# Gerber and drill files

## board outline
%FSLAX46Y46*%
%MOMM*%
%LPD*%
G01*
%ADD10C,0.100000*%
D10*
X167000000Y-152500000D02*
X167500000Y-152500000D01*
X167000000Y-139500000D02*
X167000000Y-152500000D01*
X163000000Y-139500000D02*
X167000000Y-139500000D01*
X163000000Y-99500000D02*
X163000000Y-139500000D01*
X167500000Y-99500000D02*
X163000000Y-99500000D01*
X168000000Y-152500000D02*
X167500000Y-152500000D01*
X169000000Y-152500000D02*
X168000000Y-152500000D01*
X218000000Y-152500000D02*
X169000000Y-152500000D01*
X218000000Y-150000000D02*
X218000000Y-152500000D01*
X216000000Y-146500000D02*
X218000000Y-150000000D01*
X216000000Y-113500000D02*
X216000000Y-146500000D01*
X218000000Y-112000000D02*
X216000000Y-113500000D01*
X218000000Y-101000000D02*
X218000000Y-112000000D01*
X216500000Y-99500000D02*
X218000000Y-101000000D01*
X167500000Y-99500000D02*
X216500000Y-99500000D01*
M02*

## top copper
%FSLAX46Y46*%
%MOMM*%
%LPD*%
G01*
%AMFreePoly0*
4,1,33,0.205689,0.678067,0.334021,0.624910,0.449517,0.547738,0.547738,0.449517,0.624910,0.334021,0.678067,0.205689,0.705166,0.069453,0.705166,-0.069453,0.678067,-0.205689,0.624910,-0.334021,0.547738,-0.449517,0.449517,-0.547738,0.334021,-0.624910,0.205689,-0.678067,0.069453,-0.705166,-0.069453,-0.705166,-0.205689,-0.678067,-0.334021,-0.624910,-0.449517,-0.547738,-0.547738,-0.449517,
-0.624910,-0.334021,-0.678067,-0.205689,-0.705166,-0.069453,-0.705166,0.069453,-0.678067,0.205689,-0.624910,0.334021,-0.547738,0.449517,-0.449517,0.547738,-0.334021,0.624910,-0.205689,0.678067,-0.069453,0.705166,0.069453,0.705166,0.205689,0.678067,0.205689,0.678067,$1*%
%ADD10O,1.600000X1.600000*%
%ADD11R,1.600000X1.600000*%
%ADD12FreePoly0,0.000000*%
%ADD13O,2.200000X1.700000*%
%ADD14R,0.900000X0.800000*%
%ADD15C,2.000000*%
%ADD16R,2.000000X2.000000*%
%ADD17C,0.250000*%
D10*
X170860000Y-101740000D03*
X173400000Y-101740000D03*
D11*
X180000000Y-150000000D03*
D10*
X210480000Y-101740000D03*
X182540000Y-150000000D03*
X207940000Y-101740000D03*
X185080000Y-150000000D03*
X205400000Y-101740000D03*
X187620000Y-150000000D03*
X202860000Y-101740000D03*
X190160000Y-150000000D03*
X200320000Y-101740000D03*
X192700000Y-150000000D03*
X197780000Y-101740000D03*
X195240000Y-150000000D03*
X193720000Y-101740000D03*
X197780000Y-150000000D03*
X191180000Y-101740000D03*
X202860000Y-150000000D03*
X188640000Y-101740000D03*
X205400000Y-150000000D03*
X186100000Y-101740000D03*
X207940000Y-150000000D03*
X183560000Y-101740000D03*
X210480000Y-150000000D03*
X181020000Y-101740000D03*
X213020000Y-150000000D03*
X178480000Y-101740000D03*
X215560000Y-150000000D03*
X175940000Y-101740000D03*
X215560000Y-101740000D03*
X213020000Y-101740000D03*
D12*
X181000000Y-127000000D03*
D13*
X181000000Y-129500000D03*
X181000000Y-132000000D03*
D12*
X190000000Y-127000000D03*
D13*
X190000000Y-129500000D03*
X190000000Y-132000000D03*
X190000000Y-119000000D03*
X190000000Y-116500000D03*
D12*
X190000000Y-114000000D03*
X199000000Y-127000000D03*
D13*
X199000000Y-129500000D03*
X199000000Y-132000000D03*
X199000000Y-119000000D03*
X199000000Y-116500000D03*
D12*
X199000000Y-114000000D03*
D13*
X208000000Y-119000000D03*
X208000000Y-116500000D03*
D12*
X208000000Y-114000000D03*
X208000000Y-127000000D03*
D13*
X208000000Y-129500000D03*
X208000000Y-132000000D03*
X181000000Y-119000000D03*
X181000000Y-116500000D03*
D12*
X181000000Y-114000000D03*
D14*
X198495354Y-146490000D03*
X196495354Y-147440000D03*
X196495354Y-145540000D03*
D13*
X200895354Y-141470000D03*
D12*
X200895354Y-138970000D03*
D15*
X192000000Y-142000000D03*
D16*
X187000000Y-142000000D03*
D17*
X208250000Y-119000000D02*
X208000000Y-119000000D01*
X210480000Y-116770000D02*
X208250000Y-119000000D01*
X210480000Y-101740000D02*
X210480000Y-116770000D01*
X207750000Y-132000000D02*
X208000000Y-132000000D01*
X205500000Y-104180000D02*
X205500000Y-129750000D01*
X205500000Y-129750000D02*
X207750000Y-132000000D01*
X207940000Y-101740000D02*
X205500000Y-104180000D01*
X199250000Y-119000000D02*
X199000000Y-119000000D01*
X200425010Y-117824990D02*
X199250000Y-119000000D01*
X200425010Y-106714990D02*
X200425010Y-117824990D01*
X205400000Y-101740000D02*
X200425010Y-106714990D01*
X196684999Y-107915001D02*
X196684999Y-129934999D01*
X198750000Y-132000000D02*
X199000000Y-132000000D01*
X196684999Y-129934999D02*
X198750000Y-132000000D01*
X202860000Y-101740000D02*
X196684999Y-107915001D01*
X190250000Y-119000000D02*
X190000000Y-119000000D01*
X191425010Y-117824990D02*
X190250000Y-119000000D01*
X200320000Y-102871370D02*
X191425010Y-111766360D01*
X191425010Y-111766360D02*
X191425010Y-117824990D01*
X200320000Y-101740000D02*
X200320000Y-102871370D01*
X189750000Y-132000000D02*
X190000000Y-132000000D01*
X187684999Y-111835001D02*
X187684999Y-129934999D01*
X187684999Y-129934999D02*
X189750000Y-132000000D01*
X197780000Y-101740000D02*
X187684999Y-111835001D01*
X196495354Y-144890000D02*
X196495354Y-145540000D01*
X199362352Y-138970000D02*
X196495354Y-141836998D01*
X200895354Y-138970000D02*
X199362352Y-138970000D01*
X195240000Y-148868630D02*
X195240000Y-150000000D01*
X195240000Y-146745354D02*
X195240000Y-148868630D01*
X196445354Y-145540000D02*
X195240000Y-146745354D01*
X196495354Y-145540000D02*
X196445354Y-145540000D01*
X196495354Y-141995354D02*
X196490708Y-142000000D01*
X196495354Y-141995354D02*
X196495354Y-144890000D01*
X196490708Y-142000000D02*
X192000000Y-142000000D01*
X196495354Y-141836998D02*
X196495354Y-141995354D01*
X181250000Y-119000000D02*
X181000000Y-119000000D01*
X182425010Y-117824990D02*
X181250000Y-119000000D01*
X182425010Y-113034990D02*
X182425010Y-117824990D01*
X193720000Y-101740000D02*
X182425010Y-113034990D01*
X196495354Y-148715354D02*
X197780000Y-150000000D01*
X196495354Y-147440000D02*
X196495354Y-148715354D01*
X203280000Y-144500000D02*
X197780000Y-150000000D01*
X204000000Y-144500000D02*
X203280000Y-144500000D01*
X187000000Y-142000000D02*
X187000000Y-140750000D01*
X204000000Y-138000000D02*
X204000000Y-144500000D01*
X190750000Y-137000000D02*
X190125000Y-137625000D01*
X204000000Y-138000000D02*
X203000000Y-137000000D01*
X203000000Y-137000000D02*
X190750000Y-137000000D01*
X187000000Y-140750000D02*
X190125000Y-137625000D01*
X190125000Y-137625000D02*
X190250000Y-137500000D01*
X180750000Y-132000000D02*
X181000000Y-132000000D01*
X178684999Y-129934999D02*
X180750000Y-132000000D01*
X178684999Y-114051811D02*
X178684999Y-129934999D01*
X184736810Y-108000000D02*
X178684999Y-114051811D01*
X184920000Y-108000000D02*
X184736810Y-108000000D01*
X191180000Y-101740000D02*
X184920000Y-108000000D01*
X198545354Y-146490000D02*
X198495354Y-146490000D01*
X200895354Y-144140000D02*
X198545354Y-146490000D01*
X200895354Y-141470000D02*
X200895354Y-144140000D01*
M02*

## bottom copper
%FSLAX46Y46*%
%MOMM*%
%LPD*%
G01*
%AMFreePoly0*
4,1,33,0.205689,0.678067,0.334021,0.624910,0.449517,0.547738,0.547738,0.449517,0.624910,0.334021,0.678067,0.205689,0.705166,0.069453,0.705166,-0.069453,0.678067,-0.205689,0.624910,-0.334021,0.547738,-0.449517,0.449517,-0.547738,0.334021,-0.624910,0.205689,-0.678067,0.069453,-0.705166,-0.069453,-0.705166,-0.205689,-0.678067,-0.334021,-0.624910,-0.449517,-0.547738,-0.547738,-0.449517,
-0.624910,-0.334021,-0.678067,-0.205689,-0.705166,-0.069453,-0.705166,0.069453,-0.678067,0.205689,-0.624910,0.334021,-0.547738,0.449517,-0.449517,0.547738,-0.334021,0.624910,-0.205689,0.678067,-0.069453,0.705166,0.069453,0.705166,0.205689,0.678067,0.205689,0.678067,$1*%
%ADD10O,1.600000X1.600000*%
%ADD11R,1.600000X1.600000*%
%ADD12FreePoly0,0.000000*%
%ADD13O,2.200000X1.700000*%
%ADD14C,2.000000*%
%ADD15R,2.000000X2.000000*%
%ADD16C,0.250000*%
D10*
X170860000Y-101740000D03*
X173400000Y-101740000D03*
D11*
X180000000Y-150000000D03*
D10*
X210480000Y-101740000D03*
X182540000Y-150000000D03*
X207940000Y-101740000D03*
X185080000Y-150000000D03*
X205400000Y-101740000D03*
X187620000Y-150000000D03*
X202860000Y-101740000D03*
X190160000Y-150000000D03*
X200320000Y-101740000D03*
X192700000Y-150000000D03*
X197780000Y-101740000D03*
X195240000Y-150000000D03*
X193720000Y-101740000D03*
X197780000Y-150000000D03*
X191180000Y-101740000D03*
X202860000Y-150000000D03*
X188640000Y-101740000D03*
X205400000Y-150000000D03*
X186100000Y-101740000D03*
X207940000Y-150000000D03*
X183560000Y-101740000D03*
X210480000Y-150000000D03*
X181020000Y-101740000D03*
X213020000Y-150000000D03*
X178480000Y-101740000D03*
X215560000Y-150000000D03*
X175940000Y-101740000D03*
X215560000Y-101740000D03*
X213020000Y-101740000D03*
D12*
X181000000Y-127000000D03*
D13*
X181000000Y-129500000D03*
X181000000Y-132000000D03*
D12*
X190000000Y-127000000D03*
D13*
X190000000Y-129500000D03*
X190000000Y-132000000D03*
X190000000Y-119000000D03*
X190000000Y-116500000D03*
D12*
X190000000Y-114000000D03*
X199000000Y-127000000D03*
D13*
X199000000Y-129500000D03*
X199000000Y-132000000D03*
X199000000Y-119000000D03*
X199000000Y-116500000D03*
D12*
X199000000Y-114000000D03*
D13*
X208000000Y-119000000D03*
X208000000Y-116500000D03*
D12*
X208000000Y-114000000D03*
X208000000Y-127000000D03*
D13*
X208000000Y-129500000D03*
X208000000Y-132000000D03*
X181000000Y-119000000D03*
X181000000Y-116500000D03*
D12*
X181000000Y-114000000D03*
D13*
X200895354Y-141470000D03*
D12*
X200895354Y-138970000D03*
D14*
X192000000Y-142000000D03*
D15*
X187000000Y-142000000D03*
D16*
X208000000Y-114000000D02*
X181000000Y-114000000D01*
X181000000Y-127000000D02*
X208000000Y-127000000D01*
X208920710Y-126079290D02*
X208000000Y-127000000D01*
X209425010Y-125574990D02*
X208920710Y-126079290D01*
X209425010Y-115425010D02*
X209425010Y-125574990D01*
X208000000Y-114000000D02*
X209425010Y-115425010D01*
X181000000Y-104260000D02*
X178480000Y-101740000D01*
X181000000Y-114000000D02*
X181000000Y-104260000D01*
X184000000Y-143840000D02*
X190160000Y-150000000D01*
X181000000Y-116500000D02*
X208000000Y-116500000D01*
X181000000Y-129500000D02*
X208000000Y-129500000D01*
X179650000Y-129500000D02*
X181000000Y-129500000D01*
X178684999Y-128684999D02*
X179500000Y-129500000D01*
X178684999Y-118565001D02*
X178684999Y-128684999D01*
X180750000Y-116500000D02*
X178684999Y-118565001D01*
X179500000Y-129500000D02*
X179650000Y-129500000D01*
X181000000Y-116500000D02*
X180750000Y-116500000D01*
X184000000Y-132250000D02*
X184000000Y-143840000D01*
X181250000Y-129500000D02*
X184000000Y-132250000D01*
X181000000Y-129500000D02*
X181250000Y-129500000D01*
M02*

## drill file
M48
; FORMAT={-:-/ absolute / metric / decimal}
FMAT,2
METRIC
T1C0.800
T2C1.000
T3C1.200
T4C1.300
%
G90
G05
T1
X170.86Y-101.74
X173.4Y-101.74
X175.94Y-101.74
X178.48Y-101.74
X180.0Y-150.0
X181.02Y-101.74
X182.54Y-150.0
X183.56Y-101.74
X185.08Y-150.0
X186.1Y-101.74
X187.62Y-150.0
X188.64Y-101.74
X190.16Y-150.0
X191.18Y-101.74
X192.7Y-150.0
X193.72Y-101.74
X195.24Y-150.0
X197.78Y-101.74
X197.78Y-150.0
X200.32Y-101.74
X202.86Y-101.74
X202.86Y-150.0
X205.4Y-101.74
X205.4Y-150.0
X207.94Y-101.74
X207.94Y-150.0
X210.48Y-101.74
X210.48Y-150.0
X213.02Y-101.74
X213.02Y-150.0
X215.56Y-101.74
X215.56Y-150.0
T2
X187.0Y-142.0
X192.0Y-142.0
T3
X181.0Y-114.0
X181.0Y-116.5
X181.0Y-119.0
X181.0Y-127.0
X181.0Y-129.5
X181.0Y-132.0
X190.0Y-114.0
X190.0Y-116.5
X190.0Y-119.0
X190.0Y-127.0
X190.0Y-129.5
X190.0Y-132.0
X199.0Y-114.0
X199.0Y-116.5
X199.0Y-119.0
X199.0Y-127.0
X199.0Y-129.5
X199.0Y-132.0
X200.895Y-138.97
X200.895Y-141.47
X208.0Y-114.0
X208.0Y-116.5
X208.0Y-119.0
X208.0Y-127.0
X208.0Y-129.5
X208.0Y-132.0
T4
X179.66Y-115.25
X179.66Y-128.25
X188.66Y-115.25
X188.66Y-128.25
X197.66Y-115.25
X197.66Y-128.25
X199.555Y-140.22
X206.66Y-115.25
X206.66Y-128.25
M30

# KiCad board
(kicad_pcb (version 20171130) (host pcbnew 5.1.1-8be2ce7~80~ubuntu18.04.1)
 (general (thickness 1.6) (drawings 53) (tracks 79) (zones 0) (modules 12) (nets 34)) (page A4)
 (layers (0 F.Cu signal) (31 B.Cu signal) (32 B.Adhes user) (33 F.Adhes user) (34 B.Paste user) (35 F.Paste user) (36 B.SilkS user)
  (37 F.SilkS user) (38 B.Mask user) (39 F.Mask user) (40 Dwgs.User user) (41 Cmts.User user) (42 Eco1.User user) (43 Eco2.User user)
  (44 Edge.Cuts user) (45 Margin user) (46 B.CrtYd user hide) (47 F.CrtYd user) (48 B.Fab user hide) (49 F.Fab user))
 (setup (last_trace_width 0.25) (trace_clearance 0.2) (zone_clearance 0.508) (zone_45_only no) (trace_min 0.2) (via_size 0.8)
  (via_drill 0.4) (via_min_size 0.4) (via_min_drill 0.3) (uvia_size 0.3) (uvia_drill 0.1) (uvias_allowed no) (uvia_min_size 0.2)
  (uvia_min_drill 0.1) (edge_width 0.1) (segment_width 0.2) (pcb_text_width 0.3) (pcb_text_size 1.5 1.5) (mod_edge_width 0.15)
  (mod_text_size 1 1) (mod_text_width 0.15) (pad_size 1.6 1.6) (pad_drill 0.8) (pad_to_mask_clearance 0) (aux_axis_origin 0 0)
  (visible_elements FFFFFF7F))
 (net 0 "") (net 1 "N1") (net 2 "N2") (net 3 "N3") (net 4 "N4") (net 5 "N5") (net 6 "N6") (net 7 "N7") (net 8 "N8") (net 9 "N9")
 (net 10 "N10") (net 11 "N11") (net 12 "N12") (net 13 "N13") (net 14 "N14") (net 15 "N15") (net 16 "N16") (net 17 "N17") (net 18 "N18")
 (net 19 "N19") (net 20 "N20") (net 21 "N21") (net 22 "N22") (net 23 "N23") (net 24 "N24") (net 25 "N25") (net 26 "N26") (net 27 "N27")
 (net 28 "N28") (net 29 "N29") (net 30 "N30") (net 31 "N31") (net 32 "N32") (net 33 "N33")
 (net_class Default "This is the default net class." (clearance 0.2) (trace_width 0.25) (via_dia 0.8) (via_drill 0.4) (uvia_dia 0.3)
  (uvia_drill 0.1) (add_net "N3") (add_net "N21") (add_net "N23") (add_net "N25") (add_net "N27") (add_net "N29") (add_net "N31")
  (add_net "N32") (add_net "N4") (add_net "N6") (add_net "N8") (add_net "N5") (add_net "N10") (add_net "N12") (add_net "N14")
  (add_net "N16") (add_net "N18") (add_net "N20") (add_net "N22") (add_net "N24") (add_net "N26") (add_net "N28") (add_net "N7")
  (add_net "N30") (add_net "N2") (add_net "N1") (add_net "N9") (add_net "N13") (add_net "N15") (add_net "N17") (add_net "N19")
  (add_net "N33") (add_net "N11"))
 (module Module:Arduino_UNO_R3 (layer B.Cu) (at 180 150)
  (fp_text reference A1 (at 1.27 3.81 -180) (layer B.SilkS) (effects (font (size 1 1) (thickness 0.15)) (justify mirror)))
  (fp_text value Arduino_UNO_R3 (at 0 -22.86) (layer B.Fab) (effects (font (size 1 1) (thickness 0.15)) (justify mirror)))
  (pad 32 thru_hole oval (at -9.14 -48.26 270) (size 1.6 1.6) (drill 0.8) (layers *.Cu *.Mask) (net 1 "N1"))
  (pad 31 thru_hole oval (at -6.6 -48.26 270) (size 1.6 1.6) (drill 0.8) (layers *.Cu *.Mask) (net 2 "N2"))
  (pad 1 thru_hole rect (at 0 0 270) (size 1.6 1.6) (drill 0.8) (layers *.Cu *.Mask) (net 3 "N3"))
  (pad 17 thru_hole oval (at 30.48 -48.26 270) (size 1.6 1.6) (drill 0.8) (layers *.Cu *.Mask) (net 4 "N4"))
  (pad 2 thru_hole oval (at 2.54 0 270) (size 1.6 1.6) (drill 0.8) (layers *.Cu *.Mask) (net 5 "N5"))
  (pad 18 thru_hole oval (at 27.94 -48.26 270) (size 1.6 1.6) (drill 0.8) (layers *.Cu *.Mask) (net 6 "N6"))
  (pad 3 thru_hole oval (at 5.08 0 270) (size 1.6 1.6) (drill 0.8) (layers *.Cu *.Mask) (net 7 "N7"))
  (pad 19 thru_hole oval (at 25.4 -48.26 270) (size 1.6 1.6) (drill 0.8) (layers *.Cu *.Mask) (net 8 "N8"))
  (pad 4 thru_hole oval (at 7.62 0 270) (size 1.6 1.6) (drill 0.8) (layers *.Cu *.Mask) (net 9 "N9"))
  (pad 20 thru_hole oval (at 22.86 -48.26 270) (size 1.6 1.6) (drill 0.8) (layers *.Cu *.Mask) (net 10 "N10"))
  (pad 5 thru_hole oval (at 10.16 0 270) (size 1.6 1.6) (drill 0.8) (layers *.Cu *.Mask) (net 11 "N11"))
  (pad 21 thru_hole oval (at 20.32 -48.26 270) (size 1.6 1.6) (drill 0.8) (layers *.Cu *.Mask) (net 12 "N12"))
  (pad 6 thru_hole oval (at 12.7 0 270) (size 1.6 1.6) (drill 0.8) (layers *.Cu *.Mask) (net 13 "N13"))
  (pad 22 thru_hole oval (at 17.78 -48.26 270) (size 1.6 1.6) (drill 0.8) (layers *.Cu *.Mask) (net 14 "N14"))
  (pad 7 thru_hole oval (at 15.24 0 270) (size 1.6 1.6) (drill 0.8) (layers *.Cu *.Mask) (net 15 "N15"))
  (pad 23 thru_hole oval (at 13.72 -48.26 270) (size 1.6 1.6) (drill 0.8) (layers *.Cu *.Mask) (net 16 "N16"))
  (pad 8 thru_hole oval (at 17.78 0 270) (size 1.6 1.6) (drill 0.8) (layers *.Cu *.Mask) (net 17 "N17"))
  (pad 24 thru_hole oval (at 11.18 -48.26 270) (size 1.6 1.6) (drill 0.8) (layers *.Cu *.Mask) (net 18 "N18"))
  (pad 9 thru_hole oval (at 22.86 0 270) (size 1.6 1.6) (drill 0.8) (layers *.Cu *.Mask) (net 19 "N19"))
  (pad 25 thru_hole oval (at 8.64 -48.26 270) (size 1.6 1.6) (drill 0.8) (layers *.Cu *.Mask) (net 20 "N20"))
  (pad 10 thru_hole oval (at 25.4 0 270) (size 1.6 1.6) (drill 0.8) (layers *.Cu *.Mask) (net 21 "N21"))
  (pad 26 thru_hole oval (at 6.1 -48.26 270) (size 1.6 1.6) (drill 0.8) (layers *.Cu *.Mask) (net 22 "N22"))
  (pad 11 thru_hole oval (at 27.94 0 270) (size 1.6 1.6) (drill 0.8) (layers *.Cu *.Mask) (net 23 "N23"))
  (pad 27 thru_hole oval (at 3.56 -48.26 270) (size 1.6 1.6) (drill 0.8) (layers *.Cu *.Mask) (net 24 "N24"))
  (pad 12 thru_hole oval (at 30.48 0 270) (size 1.6 1.6) (drill 0.8) (layers *.Cu *.Mask) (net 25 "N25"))
  (pad 28 thru_hole oval (at 1.02 -48.26 270) (size 1.6 1.6) (drill 0.8) (layers *.Cu *.Mask) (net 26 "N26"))
  (pad 13 thru_hole oval (at 33.02 0 270) (size 1.6 1.6) (drill 0.8) (layers *.Cu *.Mask) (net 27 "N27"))
  (pad 29 thru_hole oval (at -1.52 -48.26 270) (size 1.6 1.6) (drill 0.8) (layers *.Cu *.Mask) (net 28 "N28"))
  (pad 14 thru_hole oval (at 35.56 0 270) (size 1.6 1.6) (drill 0.8) (layers *.Cu *.Mask) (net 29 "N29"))
  (pad 30 thru_hole oval (at -4.06 -48.26 270) (size 1.6 1.6) (drill 0.8) (layers *.Cu *.Mask) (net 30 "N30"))
  (pad 15 thru_hole oval (at 35.56 -48.26 270) (size 1.6 1.6) (drill 0.8) (layers *.Cu *.Mask) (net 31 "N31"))
  (pad 16 thru_hole oval (at 33.02 -48.26 270) (size 1.6 1.6) (drill 0.8) (layers *.Cu *.Mask) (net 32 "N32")))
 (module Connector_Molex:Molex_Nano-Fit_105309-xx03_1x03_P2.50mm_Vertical (layer F.Cu) (at 181 127)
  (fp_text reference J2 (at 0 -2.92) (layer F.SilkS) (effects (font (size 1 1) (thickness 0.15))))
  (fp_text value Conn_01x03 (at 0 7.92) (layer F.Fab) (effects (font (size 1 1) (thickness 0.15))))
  (pad 1 thru_hole custom (at 0 0) (size 1.417157 1.417157) (drill 1.2) (layers *.Cu *.Mask) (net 28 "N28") (zone_connect 0)
   (options (clearance outline) (anchor circle)) (primitives))
  (pad 2 thru_hole oval (at 0 2.5) (size 2.2 1.7) (drill 1.2) (layers *.Cu *.Mask) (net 11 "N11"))
  (pad 3 thru_hole oval (at 0 5) (size 2.2 1.7) (drill 1.2) (layers *.Cu *.Mask) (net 18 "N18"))
  (pad "" np_thru_hole circle (at -1.34 1.25) (size 1.3 1.3) (drill 1.3) (layers *.Cu *.Mask)))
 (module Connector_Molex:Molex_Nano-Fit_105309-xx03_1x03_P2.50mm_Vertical (layer F.Cu) (at 190 127)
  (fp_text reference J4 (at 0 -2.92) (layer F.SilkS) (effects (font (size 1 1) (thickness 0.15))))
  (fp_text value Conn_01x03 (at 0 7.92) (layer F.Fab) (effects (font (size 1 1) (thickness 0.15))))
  (pad 1 thru_hole custom (at 0 0) (size 1.417157 1.417157) (drill 1.2) (layers *.Cu *.Mask) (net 28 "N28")
   (options (clearance outline) (anchor circle)) (primitives))
  (pad 2 thru_hole oval (at 0 2.5) (size 2.2 1.7) (drill 1.2) (layers *.Cu *.Mask) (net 11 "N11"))
  (pad 3 thru_hole oval (at 0 5) (size 2.2 1.7) (drill 1.2) (layers *.Cu *.Mask) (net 14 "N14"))
  (pad "" np_thru_hole circle (at -1.34 1.25) (size 1.3 1.3) (drill 1.3) (layers *.Cu *.Mask)))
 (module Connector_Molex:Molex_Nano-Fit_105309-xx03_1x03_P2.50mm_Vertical (layer F.Cu) (at 190 114)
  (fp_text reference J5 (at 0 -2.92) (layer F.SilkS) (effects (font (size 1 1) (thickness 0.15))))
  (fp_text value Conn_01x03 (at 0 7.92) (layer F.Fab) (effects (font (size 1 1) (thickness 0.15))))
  (pad "" np_thru_hole circle (at -1.34 1.25) (size 1.3 1.3) (drill 1.3) (layers *.Cu *.Mask))
  (pad 3 thru_hole oval (at 0 5) (size 2.2 1.7) (drill 1.2) (layers *.Cu *.Mask) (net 12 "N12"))
  (pad 2 thru_hole oval (at 0 2.5) (size 2.2 1.7) (drill 1.2) (layers *.Cu *.Mask) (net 11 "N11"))
  (pad 1 thru_hole custom (at 0 0) (size 1.417157 1.417157) (drill 1.2) (layers *.Cu *.Mask) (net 28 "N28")
   (options (clearance outline) (anchor circle)) (primitives)))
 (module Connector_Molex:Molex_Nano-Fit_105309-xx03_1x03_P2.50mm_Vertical (layer F.Cu) (at 199 127)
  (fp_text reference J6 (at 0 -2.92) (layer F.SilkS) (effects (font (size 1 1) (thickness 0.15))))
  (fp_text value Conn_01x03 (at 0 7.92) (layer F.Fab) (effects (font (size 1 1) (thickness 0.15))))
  (pad 1 thru_hole custom (at 0 0) (size 1.417157 1.417157) (drill 1.2) (layers *.Cu *.Mask) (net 28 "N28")
   (options (clearance outline) (anchor circle)) (primitives))
  (pad 2 thru_hole oval (at 0 2.5) (size 2.2 1.7) (drill 1.2) (layers *.Cu *.Mask) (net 11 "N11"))
  (pad 3 thru_hole oval (at 0 5) (size 2.2 1.7) (drill 1.2) (layers *.Cu *.Mask) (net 10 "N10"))
  (pad "" np_thru_hole circle (at -1.34 1.25) (size 1.3 1.3) (drill 1.3) (layers *.Cu *.Mask)))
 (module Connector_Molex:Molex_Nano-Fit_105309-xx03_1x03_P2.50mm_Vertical (layer F.Cu) (at 199 114)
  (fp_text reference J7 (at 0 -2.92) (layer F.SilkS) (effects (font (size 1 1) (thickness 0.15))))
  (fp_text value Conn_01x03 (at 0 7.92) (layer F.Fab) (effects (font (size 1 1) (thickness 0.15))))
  (pad "" np_thru_hole circle (at -1.34 1.25) (size 1.3 1.3) (drill 1.3) (layers *.Cu *.Mask))
  (pad 3 thru_hole oval (at 0 5) (size 2.2 1.7) (drill 1.2) (layers *.Cu *.Mask) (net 8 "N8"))
  (pad 2 thru_hole oval (at 0 2.5) (size 2.2 1.7) (drill 1.2) (layers *.Cu *.Mask) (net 11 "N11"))
  (pad 1 thru_hole custom (at 0 0) (size 1.417157 1.417157) (drill 1.2) (layers *.Cu *.Mask) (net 28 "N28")
   (options (clearance outline) (anchor circle)) (primitives)))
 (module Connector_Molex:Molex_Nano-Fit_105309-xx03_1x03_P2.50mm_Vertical (layer F.Cu) (at 208 114)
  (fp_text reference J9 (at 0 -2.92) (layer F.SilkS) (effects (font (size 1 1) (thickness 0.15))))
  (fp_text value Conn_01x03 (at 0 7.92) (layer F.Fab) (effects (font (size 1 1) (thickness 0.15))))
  (pad "" np_thru_hole circle (at -1.34 1.25) (size 1.3 1.3) (drill 1.3) (layers *.Cu *.Mask))
  (pad 3 thru_hole oval (at 0 5) (size 2.2 1.7) (drill 1.2) (layers *.Cu *.Mask) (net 4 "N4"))
  (pad 2 thru_hole oval (at 0 2.5) (size 2.2 1.7) (drill 1.2) (layers *.Cu *.Mask) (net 11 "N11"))
  (pad 1 thru_hole custom (at 0 0) (size 1.417157 1.417157) (drill 1.2) (layers *.Cu *.Mask) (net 28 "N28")
   (options (clearance outline) (anchor circle)) (primitives)))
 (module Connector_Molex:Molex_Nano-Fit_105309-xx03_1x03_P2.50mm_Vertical (layer F.Cu) (at 208 127)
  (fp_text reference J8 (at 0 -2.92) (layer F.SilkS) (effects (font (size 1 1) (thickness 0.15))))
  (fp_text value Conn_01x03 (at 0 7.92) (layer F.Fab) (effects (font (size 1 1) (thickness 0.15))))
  (pad 1 thru_hole custom (at 0 0) (size 1.417157 1.417157) (drill 1.2) (layers *.Cu *.Mask) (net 28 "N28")
   (options (clearance outline) (anchor circle)) (primitives))
  (pad 2 thru_hole oval (at 0 2.5) (size 2.2 1.7) (drill 1.2) (layers *.Cu *.Mask) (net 11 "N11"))
  (pad 3 thru_hole oval (at 0 5) (size 2.2 1.7) (drill 1.2) (layers *.Cu *.Mask) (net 6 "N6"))
  (pad "" np_thru_hole circle (at -1.34 1.25) (size 1.3 1.3) (drill 1.3) (layers *.Cu *.Mask)))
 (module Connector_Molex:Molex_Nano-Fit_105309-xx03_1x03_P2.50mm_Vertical (layer F.Cu) (at 181 114)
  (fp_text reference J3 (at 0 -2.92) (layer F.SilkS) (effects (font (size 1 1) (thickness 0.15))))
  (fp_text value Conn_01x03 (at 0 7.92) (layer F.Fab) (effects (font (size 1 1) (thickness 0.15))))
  (pad "" np_thru_hole circle (at -1.34 1.25) (size 1.3 1.3) (drill 1.3) (layers *.Cu *.Mask))
  (pad 3 thru_hole oval (at 0 5) (size 2.2 1.7) (drill 1.2) (layers *.Cu *.Mask) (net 16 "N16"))
  (pad 2 thru_hole oval (at 0 2.5) (size 2.2 1.7) (drill 1.2) (layers *.Cu *.Mask) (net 11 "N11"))
  (pad 1 thru_hole custom (at 0 0) (size 1.417157 1.417157) (drill 1.2) (layers *.Cu *.Mask) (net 28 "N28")
   (options (clearance outline) (anchor circle)) (primitives)))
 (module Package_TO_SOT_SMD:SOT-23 (layer F.Cu) (at 197.495354 146.49)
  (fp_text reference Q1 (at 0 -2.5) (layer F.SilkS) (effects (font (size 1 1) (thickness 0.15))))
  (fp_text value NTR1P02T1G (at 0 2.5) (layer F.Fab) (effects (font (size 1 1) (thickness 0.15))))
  (pad 3 smd rect (at 1 0) (size 0.9 0.8) (layers F.Cu F.Paste F.Mask) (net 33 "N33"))
  (pad 2 smd rect (at -1 0.95) (size 0.9 0.8) (layers F.Cu F.Paste F.Mask) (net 17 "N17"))
  (pad 1 smd rect (at -1 -0.95) (size 0.9 0.8) (layers F.Cu F.Paste F.Mask) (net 15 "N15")))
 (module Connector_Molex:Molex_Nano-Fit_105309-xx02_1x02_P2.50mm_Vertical (layer F.Cu) (at 200.895354 138.97)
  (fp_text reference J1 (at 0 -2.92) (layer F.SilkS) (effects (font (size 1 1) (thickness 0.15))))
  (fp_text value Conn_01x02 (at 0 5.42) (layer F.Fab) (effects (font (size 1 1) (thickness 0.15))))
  (pad "" np_thru_hole circle (at -1.34 1.25) (size 1.3 1.3) (drill 1.3) (layers *.Cu *.Mask))
  (pad 2 thru_hole oval (at 0 2.5) (size 2.2 1.7) (drill 1.2) (layers *.Cu *.Mask) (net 33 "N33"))
  (pad 1 thru_hole custom (at 0 0) (size 1.417157 1.417157) (drill 1.2) (layers *.Cu *.Mask) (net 15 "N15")
   (options (clearance outline) (anchor circle)) (primitives)))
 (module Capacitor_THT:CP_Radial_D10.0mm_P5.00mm (layer F.Cu) (at 187 142)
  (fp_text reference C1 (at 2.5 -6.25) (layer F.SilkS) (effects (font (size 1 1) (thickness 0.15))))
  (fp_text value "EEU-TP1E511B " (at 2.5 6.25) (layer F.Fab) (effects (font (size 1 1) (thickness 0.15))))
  (pad 2 thru_hole circle (at 5 0) (size 2 2) (drill 1) (layers *.Cu *.Mask) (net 15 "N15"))
  (pad 1 thru_hole rect (at 0 0) (size 2 2) (drill 1) (layers *.Cu *.Mask) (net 17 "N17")))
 (gr_line (start 167 152.5) (end 167.5 152.5) (layer Edge.Cuts) (width 0.1))
 (gr_line (start 167 139.5) (end 167 152.5) (layer Edge.Cuts) (width 0.1))
 (gr_line (start 163 139.5) (end 167 139.5) (layer Edge.Cuts) (width 0.1))
 (gr_line (start 163 99.5) (end 163 139.5) (layer Edge.Cuts) (width 0.1))
 (gr_line (start 167.5 99.5) (end 163 99.5) (layer Edge.Cuts) (width 0.1))
 (gr_line (start 168 152.5) (end 167.5 152.5) (layer Edge.Cuts) (width 0.1))
 (gr_line (start 169 152.5) (end 168 152.5) (layer Edge.Cuts) (width 0.1))
 (gr_line (start 218 152.5) (end 169 152.5) (layer Edge.Cuts) (width 0.1))
 (gr_line (start 218 150) (end 218 152.5) (layer Edge.Cuts) (width 0.1))
 (gr_line (start 216 146.5) (end 218 150) (layer Edge.Cuts) (width 0.1))
 (gr_line (start 216 113.5) (end 216 146.5) (layer Edge.Cuts) (width 0.1))
 (gr_line (start 218 112) (end 216 113.5) (layer Edge.Cuts) (width 0.1))
 (gr_line (start 218 101) (end 218 112) (layer Edge.Cuts) (width 0.1))
 (gr_line (start 216.5 99.5) (end 218 101) (layer Edge.Cuts) (width 0.1))
 (gr_line (start 167.5 99.5) (end 216.5 99.5) (layer Edge.Cuts) (width 0.1))
 (segment (start 208.25 119) (end 208 119) (width 0.25) (layer F.Cu) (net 4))
 (segment (start 210.48 116.77) (end 208.25 119) (width 0.25) (layer F.Cu) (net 4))
 (segment (start 210.48 101.74) (end 210.48 116.77) (width 0.25) (layer F.Cu) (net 4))
 (segment (start 207.75 132) (end 208 132) (width 0.25) (layer F.Cu) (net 6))
 (segment (start 205.5 104.18) (end 205.5 129.75) (width 0.25) (layer F.Cu) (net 6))
 (segment (start 205.5 129.75) (end 207.75 132) (width 0.25) (layer F.Cu) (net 6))
 (segment (start 207.94 101.74) (end 205.5 104.18) (width 0.25) (layer F.Cu) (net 6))
 (segment (start 199.25 119) (end 199 119) (width 0.25) (layer F.Cu) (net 8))
 (segment (start 200.42501 117.82499) (end 199.25 119) (width 0.25) (layer F.Cu) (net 8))
 (segment (start 200.42501 106.71499) (end 200.42501 117.82499) (width 0.25) (layer F.Cu) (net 8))
 (segment (start 205.4 101.74) (end 200.42501 106.71499) (width 0.25) (layer F.Cu) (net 8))
 (segment (start 196.684999 107.915001) (end 196.684999 129.934999) (width 0.25) (layer F.Cu) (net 10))
 (segment (start 198.75 132) (end 199 132) (width 0.25) (layer F.Cu) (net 10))
 (segment (start 196.684999 129.934999) (end 198.75 132) (width 0.25) (layer F.Cu) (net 10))
 (segment (start 202.86 101.74) (end 196.684999 107.915001) (width 0.25) (layer F.Cu) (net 10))
 (segment (start 208 114) (end 181 114) (width 0.25) (layer B.Cu) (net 28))
 (segment (start 181 127) (end 208 127) (width 0.25) (layer B.Cu) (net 28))
 (segment (start 208.92071 126.07929) (end 208 127) (width 0.25) (layer B.Cu) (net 28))
 (segment (start 209.42501 125.57499) (end 208.92071 126.07929) (width 0.25) (layer B.Cu) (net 28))
 (segment (start 209.42501 115.42501) (end 209.42501 125.57499) (width 0.25) (layer B.Cu) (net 28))
 (segment (start 208 114) (end 209.42501 115.42501) (width 0.25) (layer B.Cu) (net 28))
 (segment (start 181 104.26) (end 178.48 101.74) (width 0.25) (layer B.Cu) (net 28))
 (segment (start 181 114) (end 181 104.26) (width 0.25) (layer B.Cu) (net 28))
 (segment (start 190.25 119) (end 190 119) (width 0.25) (layer F.Cu) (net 12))
 (segment (start 191.42501 117.82499) (end 190.25 119) (width 0.25) (layer F.Cu) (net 12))
 (segment (start 200.32 102.87137) (end 191.42501 111.76636) (width 0.25) (layer F.Cu) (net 12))
 (segment (start 191.42501 111.76636) (end 191.42501 117.82499) (width 0.25) (layer F.Cu) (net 12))
 (segment (start 200.32 101.74) (end 200.32 102.87137) (width 0.25) (layer F.Cu) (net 12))
 (segment (start 189.75 132) (end 190 132) (width 0.25) (layer F.Cu) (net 14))
 (segment (start 187.684999 111.835001) (end 187.684999 129.934999) (width 0.25) (layer F.Cu) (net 14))
 (segment (start 187.684999 129.934999) (end 189.75 132) (width 0.25) (layer F.Cu) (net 14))
 (segment (start 197.78 101.74) (end 187.684999 111.835001) (width 0.25) (layer F.Cu) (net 14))
 (segment (start 196.495354 144.89) (end 196.495354 145.54) (width 0.25) (layer F.Cu) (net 15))
 (segment (start 199.362352 138.97) (end 196.495354 141.836998) (width 0.25) (layer F.Cu) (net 15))
 (segment (start 200.895354 138.97) (end 199.362352 138.97) (width 0.25) (layer F.Cu) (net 15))
 (segment (start 195.24 148.86863) (end 195.24 150) (width 0.25) (layer F.Cu) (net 15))
 (segment (start 195.24 146.745354) (end 195.24 148.86863) (width 0.25) (layer F.Cu) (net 15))
 (segment (start 196.445354 145.54) (end 195.24 146.745354) (width 0.25) (layer F.Cu) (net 15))
 (segment (start 196.495354 145.54) (end 196.445354 145.54) (width 0.25) (layer F.Cu) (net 15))
 (segment (start 196.495354 141.995354) (end 196.490708 142) (width 0.25) (layer F.Cu) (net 15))
 (segment (start 196.495354 141.995354) (end 196.495354 144.89) (width 0.25) (layer F.Cu) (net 15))
 (segment (start 196.490708 142) (end 192 142) (width 0.25) (layer F.Cu) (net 15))
 (segment (start 196.495354 141.836998) (end 196.495354 141.995354) (width 0.25) (layer F.Cu) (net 15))
 (segment (start 181.25 119) (end 181 119) (width 0.25) (layer F.Cu) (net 16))
 (segment (start 182.42501 117.82499) (end 181.25 119) (width 0.25) (layer F.Cu) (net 16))
 (segment (start 182.42501 113.03499) (end 182.42501 117.82499) (width 0.25) (layer F.Cu) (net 16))
 (segment (start 193.72 101.74) (end 182.42501 113.03499) (width 0.25) (layer F.Cu) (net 16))
 (segment (start 196.495354 148.715354) (end 197.78 150) (width 0.25) (layer F.Cu) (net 17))
 (segment (start 196.495354 147.44) (end 196.495354 148.715354) (width 0.25) (layer F.Cu) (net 17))
 (segment (start 203.28 144.5) (end 197.78 150) (width 0.25) (layer F.Cu) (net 17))
 (segment (start 204 144.5) (end 203.28 144.5) (width 0.25) (layer F.Cu) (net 17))
 (segment (start 187 142) (end 187 140.75) (width 0.25) (layer F.Cu) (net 17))
 (segment (start 204 138) (end 204 144.5) (width 0.25) (layer F.Cu) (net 17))
 (segment (start 190.75 137) (end 190.125 137.625) (width 0.25) (layer F.Cu) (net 17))
 (segment (start 204 138) (end 203 137) (width 0.25) (layer F.Cu) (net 17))
 (segment (start 203 137) (end 190.75 137) (width 0.25) (layer F.Cu) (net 17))
 (segment (start 187 140.75) (end 190.125 137.625) (width 0.25) (layer F.Cu) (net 17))
 (segment (start 190.125 137.625) (end 190.25 137.5) (width 0.25) (layer F.Cu) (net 17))
 (segment (start 180.75 132) (end 181 132) (width 0.25) (layer F.Cu) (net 18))
 (segment (start 178.684999 129.934999) (end 180.75 132) (width 0.25) (layer F.Cu) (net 18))
 (segment (start 178.684999 114.051811) (end 178.684999 129.934999) (width 0.25) (layer F.Cu) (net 18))
 (segment (start 184.73681 108) (end 178.684999 114.051811) (width 0.25) (layer F.Cu) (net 18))
 (segment (start 184.92 108) (end 184.73681 108) (width 0.25) (layer F.Cu) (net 18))
 (segment (start 191.18 101.74) (end 184.92 108) (width 0.25) (layer F.Cu) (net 18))
 (segment (start 184 143.84) (end 190.16 150) (width 0.25) (layer B.Cu) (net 11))
 (segment (start 181 116.5) (end 208 116.5) (width 0.25) (layer B.Cu) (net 11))
 (segment (start 181 129.5) (end 208 129.5) (width 0.25) (layer B.Cu) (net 11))
 (segment (start 179.65 129.5) (end 181 129.5) (width 0.25) (layer B.Cu) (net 11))
 (segment (start 178.684999 128.684999) (end 179.5 129.5) (width 0.25) (layer B.Cu) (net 11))
 (segment (start 178.684999 118.565001) (end 178.684999 128.684999) (width 0.25) (layer B.Cu) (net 11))
 (segment (start 180.75 116.5) (end 178.684999 118.565001) (width 0.25) (layer B.Cu) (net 11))
 (segment (start 179.5 129.5) (end 179.65 129.5) (width 0.25) (layer B.Cu) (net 11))
 (segment (start 181 116.5) (end 180.75 116.5) (width 0.25) (layer B.Cu) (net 11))
 (segment (start 184 132.25) (end 184 143.84) (width 0.25) (layer B.Cu) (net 11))
 (segment (start 181.25 129.5) (end 184 132.25) (width 0.25) (layer B.Cu) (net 11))
 (segment (start 181 129.5) (end 181.25 129.5) (width 0.25) (layer B.Cu) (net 11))
 (segment (start 198.545354 146.49) (end 198.495354 146.49) (width 0.25) (layer F.Cu) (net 33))
 (segment (start 200.895354 144.14) (end 198.545354 146.49) (width 0.25) (layer F.Cu) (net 33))
 (segment (start 200.895354 141.47) (end 200.895354 144.14) (width 0.25) (layer F.Cu) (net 33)))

